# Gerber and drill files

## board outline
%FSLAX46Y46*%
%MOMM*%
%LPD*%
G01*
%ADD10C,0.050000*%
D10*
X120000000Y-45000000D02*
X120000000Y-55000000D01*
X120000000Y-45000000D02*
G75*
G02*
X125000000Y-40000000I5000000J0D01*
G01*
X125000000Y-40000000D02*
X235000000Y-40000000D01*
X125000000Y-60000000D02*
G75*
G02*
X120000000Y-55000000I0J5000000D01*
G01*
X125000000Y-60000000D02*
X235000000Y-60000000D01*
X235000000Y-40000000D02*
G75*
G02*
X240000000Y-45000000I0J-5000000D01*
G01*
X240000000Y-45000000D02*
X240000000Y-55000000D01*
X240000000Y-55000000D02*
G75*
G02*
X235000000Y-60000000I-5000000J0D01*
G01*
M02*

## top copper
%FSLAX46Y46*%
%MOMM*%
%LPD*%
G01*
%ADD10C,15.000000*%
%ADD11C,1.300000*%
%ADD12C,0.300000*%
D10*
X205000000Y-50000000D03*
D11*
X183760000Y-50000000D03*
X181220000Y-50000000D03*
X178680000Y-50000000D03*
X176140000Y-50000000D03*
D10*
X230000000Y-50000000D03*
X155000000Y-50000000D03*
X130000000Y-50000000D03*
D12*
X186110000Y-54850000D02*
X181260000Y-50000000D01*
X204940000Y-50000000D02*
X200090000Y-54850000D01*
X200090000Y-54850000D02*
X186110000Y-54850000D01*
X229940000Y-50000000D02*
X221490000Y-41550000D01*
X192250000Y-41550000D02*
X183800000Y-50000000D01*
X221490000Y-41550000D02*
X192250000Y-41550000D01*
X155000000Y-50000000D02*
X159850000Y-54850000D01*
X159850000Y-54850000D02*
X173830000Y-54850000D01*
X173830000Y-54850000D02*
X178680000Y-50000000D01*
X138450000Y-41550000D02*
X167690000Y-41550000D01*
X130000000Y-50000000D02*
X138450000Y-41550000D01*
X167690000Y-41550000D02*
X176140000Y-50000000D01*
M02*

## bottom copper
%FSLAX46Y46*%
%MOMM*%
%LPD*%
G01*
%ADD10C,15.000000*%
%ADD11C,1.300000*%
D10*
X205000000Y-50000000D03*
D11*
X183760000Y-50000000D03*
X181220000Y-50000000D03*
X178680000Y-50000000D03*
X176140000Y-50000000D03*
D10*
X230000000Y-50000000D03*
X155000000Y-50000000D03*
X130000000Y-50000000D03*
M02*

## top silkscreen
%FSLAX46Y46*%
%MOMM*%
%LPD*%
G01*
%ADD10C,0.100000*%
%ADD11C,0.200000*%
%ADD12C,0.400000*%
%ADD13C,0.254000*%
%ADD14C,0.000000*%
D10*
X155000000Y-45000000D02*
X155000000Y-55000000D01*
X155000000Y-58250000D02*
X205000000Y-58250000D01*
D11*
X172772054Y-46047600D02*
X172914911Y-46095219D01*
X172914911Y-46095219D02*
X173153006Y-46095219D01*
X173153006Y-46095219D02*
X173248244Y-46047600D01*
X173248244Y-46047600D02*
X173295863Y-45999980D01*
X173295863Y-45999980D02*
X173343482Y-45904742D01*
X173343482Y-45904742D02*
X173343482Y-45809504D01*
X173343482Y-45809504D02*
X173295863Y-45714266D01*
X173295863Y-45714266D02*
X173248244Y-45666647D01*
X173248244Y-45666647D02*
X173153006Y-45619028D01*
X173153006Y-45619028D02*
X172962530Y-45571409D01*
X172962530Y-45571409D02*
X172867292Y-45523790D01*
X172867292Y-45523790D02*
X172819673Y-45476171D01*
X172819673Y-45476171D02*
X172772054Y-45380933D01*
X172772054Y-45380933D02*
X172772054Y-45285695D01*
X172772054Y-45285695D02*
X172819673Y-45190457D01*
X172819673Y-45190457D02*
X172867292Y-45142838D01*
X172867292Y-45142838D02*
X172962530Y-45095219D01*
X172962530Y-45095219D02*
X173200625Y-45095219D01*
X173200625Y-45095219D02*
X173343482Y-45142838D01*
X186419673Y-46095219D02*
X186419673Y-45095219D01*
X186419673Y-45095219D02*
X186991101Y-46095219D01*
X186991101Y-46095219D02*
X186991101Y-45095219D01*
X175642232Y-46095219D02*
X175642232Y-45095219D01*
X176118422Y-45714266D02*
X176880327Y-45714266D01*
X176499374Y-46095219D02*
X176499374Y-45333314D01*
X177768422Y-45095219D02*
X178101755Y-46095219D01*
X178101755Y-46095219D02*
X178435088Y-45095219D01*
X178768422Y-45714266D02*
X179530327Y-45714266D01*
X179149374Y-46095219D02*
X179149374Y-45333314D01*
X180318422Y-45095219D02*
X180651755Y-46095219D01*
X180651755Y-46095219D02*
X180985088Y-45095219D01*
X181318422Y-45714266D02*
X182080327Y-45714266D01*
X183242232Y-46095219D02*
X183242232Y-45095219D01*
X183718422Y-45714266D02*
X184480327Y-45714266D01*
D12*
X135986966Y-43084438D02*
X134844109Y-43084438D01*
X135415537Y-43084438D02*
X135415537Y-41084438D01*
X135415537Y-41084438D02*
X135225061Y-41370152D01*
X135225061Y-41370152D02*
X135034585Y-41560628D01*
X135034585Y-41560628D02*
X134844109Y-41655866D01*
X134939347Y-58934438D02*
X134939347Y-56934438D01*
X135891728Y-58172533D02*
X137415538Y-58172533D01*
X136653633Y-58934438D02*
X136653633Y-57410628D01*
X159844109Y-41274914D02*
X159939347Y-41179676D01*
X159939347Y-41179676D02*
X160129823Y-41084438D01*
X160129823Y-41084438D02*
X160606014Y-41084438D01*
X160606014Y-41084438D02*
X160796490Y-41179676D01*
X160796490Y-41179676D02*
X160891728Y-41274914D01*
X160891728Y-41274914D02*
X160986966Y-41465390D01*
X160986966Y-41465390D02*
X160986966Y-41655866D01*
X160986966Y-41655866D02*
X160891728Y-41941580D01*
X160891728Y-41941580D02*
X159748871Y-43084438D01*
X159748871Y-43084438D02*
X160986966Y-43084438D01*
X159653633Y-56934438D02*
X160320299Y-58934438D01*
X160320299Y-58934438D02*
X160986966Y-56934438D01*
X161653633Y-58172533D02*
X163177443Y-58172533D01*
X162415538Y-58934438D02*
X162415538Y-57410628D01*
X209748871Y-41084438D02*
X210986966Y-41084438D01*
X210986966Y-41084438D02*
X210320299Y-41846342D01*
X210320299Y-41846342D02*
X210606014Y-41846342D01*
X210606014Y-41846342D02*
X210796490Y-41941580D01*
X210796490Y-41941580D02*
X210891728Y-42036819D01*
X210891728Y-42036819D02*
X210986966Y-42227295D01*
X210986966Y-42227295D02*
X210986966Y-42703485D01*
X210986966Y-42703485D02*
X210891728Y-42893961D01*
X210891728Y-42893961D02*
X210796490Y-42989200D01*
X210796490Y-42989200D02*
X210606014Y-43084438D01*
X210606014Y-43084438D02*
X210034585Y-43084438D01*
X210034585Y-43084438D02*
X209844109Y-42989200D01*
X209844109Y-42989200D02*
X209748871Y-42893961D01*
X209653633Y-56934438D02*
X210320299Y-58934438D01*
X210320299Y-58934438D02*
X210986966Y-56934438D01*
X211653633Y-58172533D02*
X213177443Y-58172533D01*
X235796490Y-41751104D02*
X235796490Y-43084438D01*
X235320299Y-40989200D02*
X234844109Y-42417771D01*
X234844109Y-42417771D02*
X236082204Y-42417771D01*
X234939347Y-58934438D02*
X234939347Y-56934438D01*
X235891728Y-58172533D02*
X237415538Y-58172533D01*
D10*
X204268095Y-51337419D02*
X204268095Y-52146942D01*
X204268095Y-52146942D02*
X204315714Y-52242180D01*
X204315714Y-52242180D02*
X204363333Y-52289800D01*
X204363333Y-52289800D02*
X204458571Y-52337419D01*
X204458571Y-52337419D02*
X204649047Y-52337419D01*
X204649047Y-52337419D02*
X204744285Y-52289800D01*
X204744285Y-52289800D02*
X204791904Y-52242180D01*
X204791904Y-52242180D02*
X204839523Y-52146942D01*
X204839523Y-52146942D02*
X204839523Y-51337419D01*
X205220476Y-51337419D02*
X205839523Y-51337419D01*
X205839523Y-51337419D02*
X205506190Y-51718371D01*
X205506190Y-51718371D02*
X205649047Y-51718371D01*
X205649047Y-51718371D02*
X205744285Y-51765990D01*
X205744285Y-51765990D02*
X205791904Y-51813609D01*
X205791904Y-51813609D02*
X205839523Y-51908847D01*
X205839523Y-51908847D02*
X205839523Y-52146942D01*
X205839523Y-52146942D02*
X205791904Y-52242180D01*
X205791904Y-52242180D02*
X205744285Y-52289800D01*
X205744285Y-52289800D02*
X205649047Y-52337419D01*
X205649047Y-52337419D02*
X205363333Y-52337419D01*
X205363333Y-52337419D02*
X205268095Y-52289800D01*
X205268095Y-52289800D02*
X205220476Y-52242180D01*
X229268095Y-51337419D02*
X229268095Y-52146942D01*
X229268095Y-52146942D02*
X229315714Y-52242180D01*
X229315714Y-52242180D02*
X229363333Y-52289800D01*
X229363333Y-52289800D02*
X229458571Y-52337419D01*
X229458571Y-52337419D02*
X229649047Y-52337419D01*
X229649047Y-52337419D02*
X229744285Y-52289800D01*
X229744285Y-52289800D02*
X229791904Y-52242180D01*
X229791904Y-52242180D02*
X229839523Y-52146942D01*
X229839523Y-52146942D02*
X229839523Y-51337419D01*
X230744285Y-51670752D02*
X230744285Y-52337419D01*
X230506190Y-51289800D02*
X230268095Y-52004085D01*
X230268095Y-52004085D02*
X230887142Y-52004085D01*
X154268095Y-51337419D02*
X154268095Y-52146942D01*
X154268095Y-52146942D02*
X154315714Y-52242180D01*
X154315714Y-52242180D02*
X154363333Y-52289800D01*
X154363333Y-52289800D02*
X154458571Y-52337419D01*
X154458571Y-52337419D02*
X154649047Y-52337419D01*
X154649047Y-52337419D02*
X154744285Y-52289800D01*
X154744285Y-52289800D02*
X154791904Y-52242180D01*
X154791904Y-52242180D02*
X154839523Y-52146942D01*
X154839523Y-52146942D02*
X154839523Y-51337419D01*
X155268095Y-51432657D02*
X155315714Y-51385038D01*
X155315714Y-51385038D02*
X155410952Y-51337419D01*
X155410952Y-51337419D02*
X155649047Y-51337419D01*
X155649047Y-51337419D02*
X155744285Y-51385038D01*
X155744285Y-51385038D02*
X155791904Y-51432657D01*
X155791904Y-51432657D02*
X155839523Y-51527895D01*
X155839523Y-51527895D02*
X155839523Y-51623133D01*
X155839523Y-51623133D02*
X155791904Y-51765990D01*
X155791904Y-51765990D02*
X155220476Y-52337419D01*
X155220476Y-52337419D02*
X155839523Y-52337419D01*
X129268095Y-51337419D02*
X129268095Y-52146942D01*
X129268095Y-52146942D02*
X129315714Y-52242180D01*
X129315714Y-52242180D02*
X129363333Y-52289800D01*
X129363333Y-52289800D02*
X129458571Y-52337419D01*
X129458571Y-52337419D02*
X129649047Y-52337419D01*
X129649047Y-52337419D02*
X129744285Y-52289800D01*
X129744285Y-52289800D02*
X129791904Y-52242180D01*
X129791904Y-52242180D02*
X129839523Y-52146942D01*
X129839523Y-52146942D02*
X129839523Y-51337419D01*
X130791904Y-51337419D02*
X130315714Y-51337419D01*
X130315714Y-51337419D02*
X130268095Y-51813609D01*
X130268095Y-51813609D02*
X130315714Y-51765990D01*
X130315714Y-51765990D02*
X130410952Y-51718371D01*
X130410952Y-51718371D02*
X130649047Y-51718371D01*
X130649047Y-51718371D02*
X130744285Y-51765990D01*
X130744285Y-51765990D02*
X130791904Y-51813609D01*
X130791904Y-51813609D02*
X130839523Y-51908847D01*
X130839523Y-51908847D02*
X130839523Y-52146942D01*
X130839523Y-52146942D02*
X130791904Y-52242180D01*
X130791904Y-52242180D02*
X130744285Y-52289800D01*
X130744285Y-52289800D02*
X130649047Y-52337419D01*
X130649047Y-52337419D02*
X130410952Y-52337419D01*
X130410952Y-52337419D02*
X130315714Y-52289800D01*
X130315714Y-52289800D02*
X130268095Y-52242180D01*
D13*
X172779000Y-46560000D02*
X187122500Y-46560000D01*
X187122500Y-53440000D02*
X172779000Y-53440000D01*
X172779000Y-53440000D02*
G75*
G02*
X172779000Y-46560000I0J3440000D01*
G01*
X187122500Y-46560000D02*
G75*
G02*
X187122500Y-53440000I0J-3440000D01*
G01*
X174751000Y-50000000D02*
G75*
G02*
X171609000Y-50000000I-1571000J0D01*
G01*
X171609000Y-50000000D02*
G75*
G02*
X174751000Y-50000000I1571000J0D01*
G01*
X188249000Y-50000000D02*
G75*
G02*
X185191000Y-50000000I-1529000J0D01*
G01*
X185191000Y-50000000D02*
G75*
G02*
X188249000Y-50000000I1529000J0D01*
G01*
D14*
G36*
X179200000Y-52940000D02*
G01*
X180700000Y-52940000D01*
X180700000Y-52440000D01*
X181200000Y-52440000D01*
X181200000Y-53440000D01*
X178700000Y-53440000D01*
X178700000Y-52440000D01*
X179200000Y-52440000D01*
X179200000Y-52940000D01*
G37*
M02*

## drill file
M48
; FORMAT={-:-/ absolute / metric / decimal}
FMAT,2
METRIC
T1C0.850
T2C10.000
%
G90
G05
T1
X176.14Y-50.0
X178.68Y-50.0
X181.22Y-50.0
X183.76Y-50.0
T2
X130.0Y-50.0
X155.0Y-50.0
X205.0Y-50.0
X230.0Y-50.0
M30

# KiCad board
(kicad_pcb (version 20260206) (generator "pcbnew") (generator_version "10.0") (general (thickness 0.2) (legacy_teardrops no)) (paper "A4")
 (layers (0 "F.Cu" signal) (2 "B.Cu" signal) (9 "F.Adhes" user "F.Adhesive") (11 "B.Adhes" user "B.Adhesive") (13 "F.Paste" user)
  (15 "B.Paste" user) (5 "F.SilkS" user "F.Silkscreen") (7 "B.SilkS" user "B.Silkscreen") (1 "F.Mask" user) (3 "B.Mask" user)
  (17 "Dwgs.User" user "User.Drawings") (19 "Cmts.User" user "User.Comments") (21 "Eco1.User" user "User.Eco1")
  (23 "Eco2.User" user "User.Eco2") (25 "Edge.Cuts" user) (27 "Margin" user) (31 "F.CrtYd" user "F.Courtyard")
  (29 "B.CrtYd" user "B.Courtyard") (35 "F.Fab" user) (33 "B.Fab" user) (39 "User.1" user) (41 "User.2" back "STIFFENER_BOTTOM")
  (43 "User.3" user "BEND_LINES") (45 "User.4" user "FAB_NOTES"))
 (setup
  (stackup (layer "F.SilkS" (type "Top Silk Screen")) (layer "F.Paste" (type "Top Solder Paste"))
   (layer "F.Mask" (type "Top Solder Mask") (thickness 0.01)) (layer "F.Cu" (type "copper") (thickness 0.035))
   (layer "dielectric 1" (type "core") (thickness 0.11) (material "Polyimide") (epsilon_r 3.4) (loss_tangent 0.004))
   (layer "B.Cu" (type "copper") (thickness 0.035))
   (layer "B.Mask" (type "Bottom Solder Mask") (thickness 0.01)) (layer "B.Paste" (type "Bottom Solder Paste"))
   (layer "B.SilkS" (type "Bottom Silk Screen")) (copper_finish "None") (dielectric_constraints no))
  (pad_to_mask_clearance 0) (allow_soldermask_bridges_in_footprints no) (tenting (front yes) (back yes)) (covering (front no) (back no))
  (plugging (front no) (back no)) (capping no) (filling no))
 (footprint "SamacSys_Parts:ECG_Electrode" (layer "F.Cu") (at 205.03 52.38)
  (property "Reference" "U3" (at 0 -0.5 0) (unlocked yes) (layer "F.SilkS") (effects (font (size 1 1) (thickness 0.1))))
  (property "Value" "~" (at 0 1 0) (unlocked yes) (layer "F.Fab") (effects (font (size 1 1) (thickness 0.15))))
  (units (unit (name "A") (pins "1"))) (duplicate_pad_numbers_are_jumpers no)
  (pad "1" thru_hole circle (at -0.03 -2.38) (size 15 15) (drill 10) (layers "*.Cu" "*.Mask") (remove_unused_layers no) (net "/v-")))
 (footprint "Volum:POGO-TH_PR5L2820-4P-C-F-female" (layer "F.Cu") (at 179.95 50 180)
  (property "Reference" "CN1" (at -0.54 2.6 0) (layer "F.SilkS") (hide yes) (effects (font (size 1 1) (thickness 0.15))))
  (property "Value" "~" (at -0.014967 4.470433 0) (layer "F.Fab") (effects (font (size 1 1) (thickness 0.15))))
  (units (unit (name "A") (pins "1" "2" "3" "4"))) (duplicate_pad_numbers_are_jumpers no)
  (fp_line (start 7.171 3.44) (end -7.1725 3.44) (stroke (width 0.254) (type default)) (layer "F.SilkS"))
  (fp_line (start -7.1725 -3.44) (end 7.171 -3.44) (stroke (width 0.254) (type default)) (layer "F.SilkS"))
  (fp_arc (start 7.171 -3.44) (mid 10.611 0) (end 7.171 3.44) (stroke (width 0.254) (type default)) (layer "F.SilkS"))
  (fp_arc (start -7.1725 3.44) (mid -10.6125 0) (end -7.1725 -3.44) (stroke (width 0.254) (type default)) (layer "F.SilkS"))
  (fp_circle (center 6.77 0) (end 8.341 0) (stroke (width 0.254) (type default)) (fill no) (layer "F.SilkS"))
  (fp_circle (center -6.77 0) (end -5.241 0) (stroke (width 0.254) (type default)) (fill no) (layer "F.SilkS"))
  (fp_poly
   (pts (xy 1.25 -2.44) (xy 1.25 -3.44) (xy -1.25 -3.44) (xy -1.25 -2.44) (xy -0.75 -2.44) (xy -0.75 -2.94) (xy 0.75 -2.94) (xy 0.75 -2.44))
   (stroke (width 0) (type default)) (fill yes) (layer "F.SilkS"))
  (pad "1" thru_hole circle (at -3.81 0 180) (size 1.3 1.3) (drill 0.85) (layers "*.Cu" "*.Mask") (remove_unused_layers no) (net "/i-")
   (thermal_bridge_angle 90))
  (pad "2" thru_hole circle (at -1.27 0 180) (size 1.3 1.3) (drill 0.85) (layers "*.Cu" "*.Mask") (remove_unused_layers no) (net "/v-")
   (thermal_bridge_angle 90))
  (pad "3" thru_hole circle (at 1.27 0 180) (size 1.3 1.3) (drill 0.85) (layers "*.Cu" "*.Mask") (remove_unused_layers no) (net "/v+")
   (thermal_bridge_angle 90))
  (pad "4" thru_hole circle (at 3.81 0 180) (size 1.3 1.3) (drill 0.85) (layers "*.Cu" "*.Mask") (remove_unused_layers no) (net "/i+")
   (thermal_bridge_angle 90)))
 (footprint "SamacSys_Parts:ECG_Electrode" (layer "F.Cu") (at 230.03 52.38)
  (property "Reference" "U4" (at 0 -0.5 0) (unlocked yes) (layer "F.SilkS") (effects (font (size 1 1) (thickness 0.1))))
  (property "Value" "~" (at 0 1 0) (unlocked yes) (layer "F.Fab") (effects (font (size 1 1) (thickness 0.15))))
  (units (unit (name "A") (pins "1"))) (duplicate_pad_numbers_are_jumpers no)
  (pad "1" thru_hole circle (at -0.03 -2.38) (size 15 15) (drill 10) (layers "*.Cu" "*.Mask") (remove_unused_layers no) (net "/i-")))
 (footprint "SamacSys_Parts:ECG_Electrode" (layer "F.Cu") (at 155.03 52.38)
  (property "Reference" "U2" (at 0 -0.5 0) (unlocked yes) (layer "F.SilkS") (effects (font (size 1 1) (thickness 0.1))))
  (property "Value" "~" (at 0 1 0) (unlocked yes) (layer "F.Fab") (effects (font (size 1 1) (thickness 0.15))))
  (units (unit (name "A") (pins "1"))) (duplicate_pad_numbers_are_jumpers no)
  (pad "1" thru_hole circle (at -0.03 -2.38) (size 15 15) (drill 10) (layers "*.Cu" "*.Mask") (remove_unused_layers no) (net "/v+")))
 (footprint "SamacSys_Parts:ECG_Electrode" (layer "F.Cu") (at 130.03 52.38)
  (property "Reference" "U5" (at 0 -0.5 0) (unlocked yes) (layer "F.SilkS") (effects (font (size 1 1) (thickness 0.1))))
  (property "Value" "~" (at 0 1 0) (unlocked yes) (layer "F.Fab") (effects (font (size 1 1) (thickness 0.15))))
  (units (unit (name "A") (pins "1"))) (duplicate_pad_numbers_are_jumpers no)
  (pad "1" thru_hole circle (at -0.03 -2.38) (size 15 15) (drill 10) (layers "*.Cu" "*.Mask") (remove_unused_layers no) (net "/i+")))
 (gr_line (start 155 45) (end 155 55) (stroke (width 0.1) (type default)) (layer "F.SilkS"))
 (gr_line (start 155 58.25) (end 205 58.25) (stroke (width 0.1) (type default)) (layer "F.SilkS"))
 (gr_line (start 120 45) (end 120 55) (stroke (width 0.05) (type default)) (layer "Edge.Cuts"))
 (gr_arc (start 120 45) (mid 121.464466 41.464466) (end 125 40) (stroke (width 0.05) (type default)) (layer "Edge.Cuts"))
 (gr_line (start 125 40) (end 235 40) (stroke (width 0.05) (type default)) (layer "Edge.Cuts"))
 (gr_arc (start 125 60) (mid 121.464466 58.535534) (end 120 55) (stroke (width 0.05) (type default)) (layer "Edge.Cuts"))
 (gr_line (start 125 60) (end 235 60) (stroke (width 0.05) (type default)) (layer "Edge.Cuts"))
 (gr_arc (start 235 40) (mid 238.535534 41.464466) (end 240 45) (stroke (width 0.05) (type default)) (layer "Edge.Cuts"))
 (gr_line (start 240 45) (end 240 55) (stroke (width 0.05) (type default)) (layer "Edge.Cuts"))
 (gr_arc (start 240 55) (mid 238.535534 58.535534) (end 235 60) (stroke (width 0.05) (type default)) (layer "Edge.Cuts"))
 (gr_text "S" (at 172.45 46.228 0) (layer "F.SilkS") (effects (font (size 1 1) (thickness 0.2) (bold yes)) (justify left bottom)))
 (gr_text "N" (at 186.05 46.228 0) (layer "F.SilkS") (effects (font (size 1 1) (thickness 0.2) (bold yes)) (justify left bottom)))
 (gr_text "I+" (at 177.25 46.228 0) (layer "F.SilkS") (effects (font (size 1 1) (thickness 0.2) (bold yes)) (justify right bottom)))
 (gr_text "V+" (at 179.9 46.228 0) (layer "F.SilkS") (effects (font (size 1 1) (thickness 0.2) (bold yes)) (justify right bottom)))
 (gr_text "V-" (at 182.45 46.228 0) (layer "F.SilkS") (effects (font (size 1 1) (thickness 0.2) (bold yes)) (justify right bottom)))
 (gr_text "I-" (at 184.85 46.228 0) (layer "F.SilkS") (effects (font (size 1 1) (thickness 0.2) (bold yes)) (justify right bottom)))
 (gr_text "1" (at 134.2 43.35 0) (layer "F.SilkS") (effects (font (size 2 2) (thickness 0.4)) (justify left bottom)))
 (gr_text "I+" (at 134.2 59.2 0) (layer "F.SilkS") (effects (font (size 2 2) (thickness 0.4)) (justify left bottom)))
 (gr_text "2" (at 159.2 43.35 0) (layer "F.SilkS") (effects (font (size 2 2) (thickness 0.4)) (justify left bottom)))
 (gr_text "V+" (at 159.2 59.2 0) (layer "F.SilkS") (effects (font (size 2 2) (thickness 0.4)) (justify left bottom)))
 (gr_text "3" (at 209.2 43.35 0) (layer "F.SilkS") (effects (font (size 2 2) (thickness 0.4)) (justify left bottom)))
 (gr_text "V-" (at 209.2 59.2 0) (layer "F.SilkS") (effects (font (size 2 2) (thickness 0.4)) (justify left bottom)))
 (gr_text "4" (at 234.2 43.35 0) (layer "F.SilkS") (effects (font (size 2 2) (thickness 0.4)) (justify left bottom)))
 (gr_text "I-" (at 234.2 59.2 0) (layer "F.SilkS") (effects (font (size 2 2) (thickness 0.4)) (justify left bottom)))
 (segment (start 186.11 54.85) (end 181.26 50) (width 0.3) (layer "F.Cu") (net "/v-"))
 (segment (start 204.94 50) (end 200.09 54.85) (width 0.3) (layer "F.Cu") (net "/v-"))
 (segment (start 200.09 54.85) (end 186.11 54.85) (width 0.3) (layer "F.Cu") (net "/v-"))
 (segment (start 229.94 50) (end 221.49 41.55) (width 0.3) (layer "F.Cu") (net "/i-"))
 (segment (start 192.25 41.55) (end 183.8 50) (width 0.3) (layer "F.Cu") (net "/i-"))
 (segment (start 221.49 41.55) (end 192.25 41.55) (width 0.3) (layer "F.Cu") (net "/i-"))
 (segment (start 155 50) (end 159.85 54.85) (width 0.3) (layer "F.Cu") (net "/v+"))
 (segment (start 159.85 54.85) (end 173.83 54.85) (width 0.3) (layer "F.Cu") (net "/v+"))
 (segment (start 173.83 54.85) (end 178.68 50) (width 0.3) (layer "F.Cu") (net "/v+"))
 (segment (start 138.45 41.55) (end 167.69 41.55) (width 0.3) (layer "F.Cu") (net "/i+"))
 (segment (start 130 50) (end 138.45 41.55) (width 0.3) (layer "F.Cu") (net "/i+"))
 (segment (start 167.69 41.55) (end 176.14 50) (width 0.3) (layer "F.Cu") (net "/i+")))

